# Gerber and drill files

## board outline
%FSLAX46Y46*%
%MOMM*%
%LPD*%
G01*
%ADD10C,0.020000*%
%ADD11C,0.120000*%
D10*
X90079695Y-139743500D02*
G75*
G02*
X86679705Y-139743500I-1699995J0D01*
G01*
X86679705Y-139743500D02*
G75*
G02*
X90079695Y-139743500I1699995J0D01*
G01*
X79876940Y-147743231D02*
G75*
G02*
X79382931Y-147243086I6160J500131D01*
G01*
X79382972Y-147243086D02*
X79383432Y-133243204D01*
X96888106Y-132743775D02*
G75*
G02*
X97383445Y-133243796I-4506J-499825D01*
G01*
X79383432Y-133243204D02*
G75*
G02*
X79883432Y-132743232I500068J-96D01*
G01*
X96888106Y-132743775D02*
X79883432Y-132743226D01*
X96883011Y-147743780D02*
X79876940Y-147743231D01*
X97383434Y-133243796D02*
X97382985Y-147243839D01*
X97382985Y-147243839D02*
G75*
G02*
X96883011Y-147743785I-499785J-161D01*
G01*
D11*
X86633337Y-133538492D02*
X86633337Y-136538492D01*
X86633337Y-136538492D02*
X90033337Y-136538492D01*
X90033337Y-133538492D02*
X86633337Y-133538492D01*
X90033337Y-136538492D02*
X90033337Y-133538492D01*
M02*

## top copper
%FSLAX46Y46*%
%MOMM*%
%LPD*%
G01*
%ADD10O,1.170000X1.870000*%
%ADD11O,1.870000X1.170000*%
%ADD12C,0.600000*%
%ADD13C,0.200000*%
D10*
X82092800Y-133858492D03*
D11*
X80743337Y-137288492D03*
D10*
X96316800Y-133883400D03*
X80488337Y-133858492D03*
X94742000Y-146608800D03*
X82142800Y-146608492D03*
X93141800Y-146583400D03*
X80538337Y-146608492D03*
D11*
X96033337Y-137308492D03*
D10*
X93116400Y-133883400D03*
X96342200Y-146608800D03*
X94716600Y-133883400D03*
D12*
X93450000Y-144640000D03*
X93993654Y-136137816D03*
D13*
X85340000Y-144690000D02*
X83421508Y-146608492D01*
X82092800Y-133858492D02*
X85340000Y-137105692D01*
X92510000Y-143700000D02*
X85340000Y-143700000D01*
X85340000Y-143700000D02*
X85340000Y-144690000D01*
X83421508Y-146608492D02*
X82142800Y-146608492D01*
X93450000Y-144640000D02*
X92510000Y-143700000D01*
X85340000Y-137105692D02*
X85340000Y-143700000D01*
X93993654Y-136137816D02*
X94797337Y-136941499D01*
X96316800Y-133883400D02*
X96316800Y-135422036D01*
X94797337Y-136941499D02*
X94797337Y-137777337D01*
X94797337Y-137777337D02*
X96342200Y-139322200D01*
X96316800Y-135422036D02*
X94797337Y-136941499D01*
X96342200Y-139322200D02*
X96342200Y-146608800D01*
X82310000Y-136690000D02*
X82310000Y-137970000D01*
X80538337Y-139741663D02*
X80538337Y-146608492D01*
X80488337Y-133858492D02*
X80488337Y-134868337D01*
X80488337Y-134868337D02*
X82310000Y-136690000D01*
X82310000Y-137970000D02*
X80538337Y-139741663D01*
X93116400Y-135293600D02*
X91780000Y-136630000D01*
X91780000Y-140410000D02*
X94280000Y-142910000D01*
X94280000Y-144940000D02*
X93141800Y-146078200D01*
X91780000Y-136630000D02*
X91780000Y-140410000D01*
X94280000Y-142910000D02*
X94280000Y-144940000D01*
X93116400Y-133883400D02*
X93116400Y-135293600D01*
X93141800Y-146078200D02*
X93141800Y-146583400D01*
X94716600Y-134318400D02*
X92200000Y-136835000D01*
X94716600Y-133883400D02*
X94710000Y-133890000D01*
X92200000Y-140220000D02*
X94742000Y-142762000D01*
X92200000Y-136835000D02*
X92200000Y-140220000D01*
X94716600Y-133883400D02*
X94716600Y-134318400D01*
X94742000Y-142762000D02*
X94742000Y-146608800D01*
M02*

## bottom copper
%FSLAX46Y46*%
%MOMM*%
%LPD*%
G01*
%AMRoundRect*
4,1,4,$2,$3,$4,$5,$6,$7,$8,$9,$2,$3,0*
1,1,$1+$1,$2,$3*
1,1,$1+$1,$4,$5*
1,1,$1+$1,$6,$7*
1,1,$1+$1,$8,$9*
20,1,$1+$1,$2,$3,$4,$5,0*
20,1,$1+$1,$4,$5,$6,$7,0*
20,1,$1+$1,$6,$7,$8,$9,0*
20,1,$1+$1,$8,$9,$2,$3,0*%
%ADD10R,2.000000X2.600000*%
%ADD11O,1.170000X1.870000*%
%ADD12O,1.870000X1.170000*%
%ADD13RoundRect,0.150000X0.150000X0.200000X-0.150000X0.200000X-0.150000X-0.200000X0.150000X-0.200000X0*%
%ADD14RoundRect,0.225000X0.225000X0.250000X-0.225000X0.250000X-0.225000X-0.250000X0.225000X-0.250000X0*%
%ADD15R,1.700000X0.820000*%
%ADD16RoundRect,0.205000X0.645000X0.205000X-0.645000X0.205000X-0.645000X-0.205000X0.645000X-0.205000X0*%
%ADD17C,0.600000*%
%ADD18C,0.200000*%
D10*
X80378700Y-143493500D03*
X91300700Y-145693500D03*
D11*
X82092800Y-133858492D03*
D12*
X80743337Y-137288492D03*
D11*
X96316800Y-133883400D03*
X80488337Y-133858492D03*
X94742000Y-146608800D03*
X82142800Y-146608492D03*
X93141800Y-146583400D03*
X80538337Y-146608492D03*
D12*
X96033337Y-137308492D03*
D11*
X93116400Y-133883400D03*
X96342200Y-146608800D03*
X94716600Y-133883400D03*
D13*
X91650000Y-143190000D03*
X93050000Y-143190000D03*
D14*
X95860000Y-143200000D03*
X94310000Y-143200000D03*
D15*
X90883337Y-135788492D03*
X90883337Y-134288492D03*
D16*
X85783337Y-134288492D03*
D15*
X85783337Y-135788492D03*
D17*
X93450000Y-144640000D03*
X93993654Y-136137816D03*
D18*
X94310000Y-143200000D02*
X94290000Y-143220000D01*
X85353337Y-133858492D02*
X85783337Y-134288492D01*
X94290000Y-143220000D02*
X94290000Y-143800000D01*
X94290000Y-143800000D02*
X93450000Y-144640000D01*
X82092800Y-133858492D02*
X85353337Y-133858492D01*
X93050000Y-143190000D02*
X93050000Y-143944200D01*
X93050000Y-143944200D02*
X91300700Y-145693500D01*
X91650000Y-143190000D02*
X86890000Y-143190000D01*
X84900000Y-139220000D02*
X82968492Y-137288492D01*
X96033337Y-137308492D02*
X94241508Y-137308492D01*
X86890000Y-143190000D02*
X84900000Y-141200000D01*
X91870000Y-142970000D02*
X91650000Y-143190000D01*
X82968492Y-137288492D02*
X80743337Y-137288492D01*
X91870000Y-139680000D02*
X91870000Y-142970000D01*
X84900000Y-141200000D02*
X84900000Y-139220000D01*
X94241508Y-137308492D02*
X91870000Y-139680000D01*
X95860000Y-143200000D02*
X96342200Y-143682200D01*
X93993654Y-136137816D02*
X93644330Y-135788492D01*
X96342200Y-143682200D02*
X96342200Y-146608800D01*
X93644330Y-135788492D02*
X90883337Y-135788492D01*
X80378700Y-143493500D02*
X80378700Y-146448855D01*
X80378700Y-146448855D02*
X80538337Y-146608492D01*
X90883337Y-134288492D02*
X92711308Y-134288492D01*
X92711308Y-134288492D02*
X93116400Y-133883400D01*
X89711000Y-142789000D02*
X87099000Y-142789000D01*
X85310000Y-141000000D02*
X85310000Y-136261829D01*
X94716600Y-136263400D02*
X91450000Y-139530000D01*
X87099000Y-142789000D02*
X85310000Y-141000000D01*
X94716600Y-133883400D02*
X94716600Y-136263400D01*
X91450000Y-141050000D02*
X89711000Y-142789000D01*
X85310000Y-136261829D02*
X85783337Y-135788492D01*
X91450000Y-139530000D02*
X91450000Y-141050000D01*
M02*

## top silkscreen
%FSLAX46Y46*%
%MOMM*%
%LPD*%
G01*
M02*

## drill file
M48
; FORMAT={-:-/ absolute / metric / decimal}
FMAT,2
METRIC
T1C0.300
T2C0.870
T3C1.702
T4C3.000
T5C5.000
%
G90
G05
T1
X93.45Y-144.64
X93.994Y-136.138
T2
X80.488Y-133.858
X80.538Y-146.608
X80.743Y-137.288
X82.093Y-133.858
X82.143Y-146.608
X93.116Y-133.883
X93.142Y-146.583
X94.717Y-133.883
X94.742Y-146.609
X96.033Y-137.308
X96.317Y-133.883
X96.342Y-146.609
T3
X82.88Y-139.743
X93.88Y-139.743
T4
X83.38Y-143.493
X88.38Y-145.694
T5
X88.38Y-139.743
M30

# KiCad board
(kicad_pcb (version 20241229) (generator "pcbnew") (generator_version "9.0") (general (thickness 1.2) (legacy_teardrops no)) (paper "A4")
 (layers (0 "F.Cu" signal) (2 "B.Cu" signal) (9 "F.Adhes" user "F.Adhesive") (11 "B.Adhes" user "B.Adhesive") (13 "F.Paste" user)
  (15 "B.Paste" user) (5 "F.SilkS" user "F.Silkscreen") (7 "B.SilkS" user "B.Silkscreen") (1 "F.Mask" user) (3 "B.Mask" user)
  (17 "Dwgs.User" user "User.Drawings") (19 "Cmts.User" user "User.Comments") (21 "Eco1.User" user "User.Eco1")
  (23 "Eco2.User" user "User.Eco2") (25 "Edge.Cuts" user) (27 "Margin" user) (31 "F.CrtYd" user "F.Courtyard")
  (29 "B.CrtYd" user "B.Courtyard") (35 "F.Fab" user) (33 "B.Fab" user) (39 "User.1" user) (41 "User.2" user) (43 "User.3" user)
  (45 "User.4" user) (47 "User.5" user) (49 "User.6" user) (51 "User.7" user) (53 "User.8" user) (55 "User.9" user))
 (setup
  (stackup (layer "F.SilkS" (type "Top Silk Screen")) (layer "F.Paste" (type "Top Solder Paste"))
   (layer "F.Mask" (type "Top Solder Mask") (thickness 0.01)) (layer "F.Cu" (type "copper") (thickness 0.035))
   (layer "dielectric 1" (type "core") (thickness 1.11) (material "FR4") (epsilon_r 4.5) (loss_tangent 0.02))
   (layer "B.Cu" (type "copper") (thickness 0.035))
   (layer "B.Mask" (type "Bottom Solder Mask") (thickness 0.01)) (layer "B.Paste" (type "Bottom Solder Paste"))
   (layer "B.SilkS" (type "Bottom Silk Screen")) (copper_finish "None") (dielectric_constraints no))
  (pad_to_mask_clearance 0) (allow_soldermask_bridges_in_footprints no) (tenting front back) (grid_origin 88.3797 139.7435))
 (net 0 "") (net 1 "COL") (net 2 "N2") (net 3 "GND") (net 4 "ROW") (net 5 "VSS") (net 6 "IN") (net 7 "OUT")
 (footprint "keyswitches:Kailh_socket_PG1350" (layer "F.Cu") (at 88.3797 139.7435)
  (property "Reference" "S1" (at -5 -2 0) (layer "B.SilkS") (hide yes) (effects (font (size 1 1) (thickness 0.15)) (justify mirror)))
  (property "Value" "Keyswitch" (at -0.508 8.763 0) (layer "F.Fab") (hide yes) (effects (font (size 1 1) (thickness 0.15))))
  (pad "" np_thru_hole circle (at -5.5 0) (size 1.7018 1.7018) (drill 1.7018) (layers "*.Cu" "*.Mask"))
  (pad "" np_thru_hole circle (at -5 3.75) (size 3 3) (drill 3) (layers "*.Cu" "*.Mask"))
  (pad "" np_thru_hole circle (at 0 0) (size 5 5) (drill 5) (layers "*.Cu" "*.Mask"))
  (pad "" np_thru_hole circle (at 0 5.95) (size 3 3) (drill 3) (layers "*.Cu" "*.Mask"))
  (pad "" np_thru_hole circle (at 5.5 0) (size 1.7018 1.7018) (drill 1.7018) (layers "*.Cu" "*.Mask"))
  (pad "1" smd rect (at -8.001 3.75) (size 2 2.6) (layers "B.Cu" "B.Mask" "B.Paste") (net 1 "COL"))
  (pad "2" smd rect (at 2.921 5.95) (size 2 2.6) (layers "B.Cu" "B.Mask" "B.Paste") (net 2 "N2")))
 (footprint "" (layer "F.Cu") (at 82.0928 133.858492 90)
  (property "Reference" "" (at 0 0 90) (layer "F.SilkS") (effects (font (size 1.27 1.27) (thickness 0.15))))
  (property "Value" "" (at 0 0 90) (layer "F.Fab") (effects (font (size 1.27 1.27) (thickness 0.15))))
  (pad "" thru_hole oval (at 0 0 180) (size 1.17 1.87) (drill 0.87) (layers "*.Cu" "*.Mask") (remove_unused_layers no) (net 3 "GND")))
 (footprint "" (layer "F.Cu") (at 80.743337 137.288492 180)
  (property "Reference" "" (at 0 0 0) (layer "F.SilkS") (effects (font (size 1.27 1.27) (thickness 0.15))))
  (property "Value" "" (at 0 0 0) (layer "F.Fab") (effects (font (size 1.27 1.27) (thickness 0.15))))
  (pad "" thru_hole oval (at 0 0 270) (size 1.17 1.87) (drill 0.87) (layers "*.Cu" "*.Mask") (remove_unused_layers no) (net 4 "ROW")))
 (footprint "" (layer "F.Cu") (at 96.3168 133.8834)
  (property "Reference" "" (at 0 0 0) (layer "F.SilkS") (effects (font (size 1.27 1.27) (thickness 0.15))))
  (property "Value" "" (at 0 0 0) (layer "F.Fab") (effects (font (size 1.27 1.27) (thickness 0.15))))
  (pad "" thru_hole oval (at 0 0 180) (size 1.17 1.87) (drill 0.87) (layers "*.Cu" "*.Mask") (remove_unused_layers no) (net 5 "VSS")))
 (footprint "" (layer "F.Cu") (at 80.488337 133.858492)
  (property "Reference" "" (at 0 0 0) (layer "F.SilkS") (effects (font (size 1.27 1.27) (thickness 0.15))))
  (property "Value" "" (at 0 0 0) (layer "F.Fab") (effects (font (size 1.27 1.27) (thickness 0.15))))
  (pad "" thru_hole oval (at 0 0 180) (size 1.17 1.87) (drill 0.87) (layers "*.Cu" "*.Mask") (remove_unused_layers no) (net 1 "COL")))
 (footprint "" (layer "F.Cu") (at 94.742 146.6088)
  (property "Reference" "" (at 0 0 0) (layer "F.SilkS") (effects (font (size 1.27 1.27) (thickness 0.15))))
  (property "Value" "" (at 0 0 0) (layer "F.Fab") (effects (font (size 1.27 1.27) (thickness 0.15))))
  (pad "" thru_hole oval (at 0 0 180) (size 1.17 1.87) (drill 0.87) (layers "*.Cu" "*.Mask") (remove_unused_layers no) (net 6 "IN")))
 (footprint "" (layer "F.Cu") (at 82.1428 146.608492 90)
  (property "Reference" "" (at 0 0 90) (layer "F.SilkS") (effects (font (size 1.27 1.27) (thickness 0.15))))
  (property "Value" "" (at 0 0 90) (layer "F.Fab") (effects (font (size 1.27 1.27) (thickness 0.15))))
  (pad "" thru_hole oval (at 0 0 180) (size 1.17 1.87) (drill 0.87) (layers "*.Cu" "*.Mask") (remove_unused_layers no) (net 3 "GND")))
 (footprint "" (layer "F.Cu") (at 93.1418 146.5834)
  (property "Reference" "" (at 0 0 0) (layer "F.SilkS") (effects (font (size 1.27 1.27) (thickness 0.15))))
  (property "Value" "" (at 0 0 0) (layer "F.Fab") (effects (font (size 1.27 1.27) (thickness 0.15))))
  (pad "" thru_hole oval (at 0 0 180) (size 1.17 1.87) (drill 0.87) (layers "*.Cu" "*.Mask") (remove_unused_layers no) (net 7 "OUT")))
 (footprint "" (layer "F.Cu") (at 80.538337 146.608492)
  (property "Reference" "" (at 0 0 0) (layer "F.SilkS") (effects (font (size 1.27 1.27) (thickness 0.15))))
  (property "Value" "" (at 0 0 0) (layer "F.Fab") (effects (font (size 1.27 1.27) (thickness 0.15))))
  (pad "" thru_hole oval (at 0 0 180) (size 1.17 1.87) (drill 0.87) (layers "*.Cu" "*.Mask") (remove_unused_layers no) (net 1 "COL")))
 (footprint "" (layer "F.Cu") (at 96.033337 137.308492 180)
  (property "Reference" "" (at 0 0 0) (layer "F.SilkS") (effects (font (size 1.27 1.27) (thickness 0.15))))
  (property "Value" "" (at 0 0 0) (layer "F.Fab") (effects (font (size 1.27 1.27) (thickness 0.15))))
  (pad "" thru_hole oval (at 0 0 270) (size 1.17 1.87) (drill 0.87) (layers "*.Cu" "*.Mask") (remove_unused_layers no) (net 4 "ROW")))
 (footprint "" (layer "F.Cu") (at 93.1164 133.8834)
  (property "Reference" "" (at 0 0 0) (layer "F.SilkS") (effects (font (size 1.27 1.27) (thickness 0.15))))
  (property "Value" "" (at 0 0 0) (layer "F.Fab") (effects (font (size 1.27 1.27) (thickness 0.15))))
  (pad "" thru_hole oval (at 0 0 180) (size 1.17 1.87) (drill 0.87) (layers "*.Cu" "*.Mask") (remove_unused_layers no) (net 7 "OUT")))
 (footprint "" (layer "F.Cu") (at 96.3422 146.6088)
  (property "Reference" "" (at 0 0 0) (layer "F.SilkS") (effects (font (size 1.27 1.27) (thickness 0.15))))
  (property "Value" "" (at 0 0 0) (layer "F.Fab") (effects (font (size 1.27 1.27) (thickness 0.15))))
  (pad "" thru_hole oval (at 0 0 180) (size 1.17 1.87) (drill 0.87) (layers "*.Cu" "*.Mask") (remove_unused_layers no) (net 5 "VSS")))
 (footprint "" (layer "F.Cu") (at 94.7166 133.8834)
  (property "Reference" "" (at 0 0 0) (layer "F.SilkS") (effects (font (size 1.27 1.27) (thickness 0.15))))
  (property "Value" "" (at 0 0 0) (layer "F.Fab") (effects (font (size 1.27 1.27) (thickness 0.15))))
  (pad "" thru_hole oval (at 0 0 180) (size 1.17 1.87) (drill 0.87) (layers "*.Cu" "*.Mask") (remove_unused_layers no) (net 6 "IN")))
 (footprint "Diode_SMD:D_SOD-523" (layer "B.Cu") (at 92.35 143.19)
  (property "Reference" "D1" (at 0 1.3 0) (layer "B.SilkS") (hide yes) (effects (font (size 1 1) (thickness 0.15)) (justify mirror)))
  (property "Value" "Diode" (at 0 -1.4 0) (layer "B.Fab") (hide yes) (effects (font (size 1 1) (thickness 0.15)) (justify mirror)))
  (pad "1" smd roundrect (at -0.7 0 180) (size 0.6 0.7) (layers "B.Cu" "B.Mask" "B.Paste") (roundrect_rratio 0.25) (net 4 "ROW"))
  (pad "2" smd roundrect (at 0.7 0 180) (size 0.6 0.7) (layers "B.Cu" "B.Mask" "B.Paste") (roundrect_rratio 0.25) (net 2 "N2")))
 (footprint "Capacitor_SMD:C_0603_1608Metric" (layer "B.Cu") (at 95.085 143.2 180)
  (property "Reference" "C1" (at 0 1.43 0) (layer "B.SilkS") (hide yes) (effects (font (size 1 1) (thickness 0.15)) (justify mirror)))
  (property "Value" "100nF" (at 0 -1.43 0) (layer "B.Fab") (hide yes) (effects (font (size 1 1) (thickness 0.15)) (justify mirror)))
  (pad "1" smd roundrect (at -0.775 0 180) (size 0.9 0.95) (layers "B.Cu" "B.Mask" "B.Paste") (roundrect_rratio 0.25) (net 5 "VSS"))
  (pad "2" smd roundrect (at 0.775 0 180) (size 0.9 0.95) (layers "B.Cu" "B.Mask" "B.Paste") (roundrect_rratio 0.25) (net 3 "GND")))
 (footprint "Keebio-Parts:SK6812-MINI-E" (layer "B.Cu") (at 88.333337 135.038492 180)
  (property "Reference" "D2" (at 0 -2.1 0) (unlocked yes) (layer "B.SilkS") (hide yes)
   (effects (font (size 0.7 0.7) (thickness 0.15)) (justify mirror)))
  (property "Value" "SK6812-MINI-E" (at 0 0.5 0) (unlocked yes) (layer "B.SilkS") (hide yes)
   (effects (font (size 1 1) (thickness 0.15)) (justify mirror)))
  (fp_line (start 1.7 1.5) (end 1.7 -1.5) (stroke (width 0.12) (type solid)) (layer "Edge.Cuts"))
  (fp_line (start 1.7 -1.5) (end -1.7 -1.5) (stroke (width 0.12) (type solid)) (layer "Edge.Cuts"))
  (fp_line (start -1.7 1.5) (end 1.7 1.5) (stroke (width 0.12) (type solid)) (layer "Edge.Cuts"))
  (fp_line (start -1.7 -1.5) (end -1.7 1.5) (stroke (width 0.12) (type solid)) (layer "Edge.Cuts"))
  (pad "1" smd rect (at -2.55 -0.75 180) (size 1.7 0.82) (layers "B.Cu" "B.Mask" "B.Paste") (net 5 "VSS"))
  (pad "2" smd rect (at -2.55 0.75 180) (size 1.7 0.82) (layers "B.Cu" "B.Mask" "B.Paste") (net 7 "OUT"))
  (pad "3" smd roundrect (at 2.55 0.75 180) (size 1.7 0.82) (layers "B.Cu" "B.Mask" "B.Paste") (roundrect_rratio 0.25) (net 3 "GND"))
  (pad "4" smd rect (at 2.55 -0.75 180) (size 1.7 0.82) (layers "B.Cu" "B.Mask" "B.Paste") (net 6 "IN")))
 (gr_circle (center 88.3797 139.7435) (end 90.068769 139.551067) (stroke (width 0.02) (type default)) (fill no) (layer "Edge.Cuts"))
 (gr_arc (start 79.87694 147.743231) (mid 79.527287 147.594577) (end 79.382972 147.243086) (stroke (width 0.02) (type default))
  (layer "Edge.Cuts"))
 (gr_line (start 79.382972 147.243086) (end 79.383432 133.243204) (stroke (width 0.02) (type default)) (layer "Edge.Cuts"))
 (gr_arc (start 96.888106 132.743775) (mid 97.238703 132.891822) (end 97.383434 133.243796) (stroke (width 0.02) (type default))
  (layer "Edge.Cuts"))
 (gr_arc (start 79.383432 133.243204) (mid 79.529908 132.889689) (end 79.883432 132.743226) (stroke (width 0.02) (type default))
  (layer "Edge.Cuts"))
 (gr_line (start 96.888106 132.743775) (end 79.883432 132.743226) (stroke (width 0.02) (type default)) (layer "Edge.Cuts"))
 (gr_line (start 96.883011 147.74378) (end 79.87694 147.743231) (stroke (width 0.02) (type default)) (layer "Edge.Cuts"))
 (gr_line (start 97.383434 133.243796) (end 97.382985 147.243839) (stroke (width 0.02) (type default)) (layer "Edge.Cuts"))
 (gr_arc (start 97.382985 147.243839) (mid 97.236591 147.597411) (end 96.883011 147.74378) (stroke (width 0.02) (type default))
  (layer "Edge.Cuts"))
 (segment (start 85.34 144.69) (end 83.421508 146.608492) (width 0.2) (layer "F.Cu") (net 3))
 (segment (start 82.0928 133.858492) (end 85.34 137.105692) (width 0.2) (layer "F.Cu") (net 3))
 (segment (start 92.51 143.7) (end 85.34 143.7) (width 0.2) (layer "F.Cu") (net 3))
 (segment (start 85.34 143.7) (end 85.34 144.69) (width 0.2) (layer "F.Cu") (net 3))
 (segment (start 83.421508 146.608492) (end 82.1428 146.608492) (width 0.2) (layer "F.Cu") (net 3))
 (segment (start 93.45 144.64) (end 92.51 143.7) (width 0.2) (layer "F.Cu") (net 3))
 (segment (start 85.34 137.105692) (end 85.34 143.7) (width 0.2) (layer "F.Cu") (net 3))
 (via (at 93.45 144.64) (size 0.6) (drill 0.3) (layers "F.Cu" "B.Cu") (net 3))
 (segment (start 94.31 143.2) (end 94.29 143.22) (width 0.2) (layer "B.Cu") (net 3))
 (segment (start 85.353337 133.858492) (end 85.783337 134.288492) (width 0.2) (layer "B.Cu") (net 3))
 (segment (start 94.29 143.22) (end 94.29 143.8) (width 0.2) (layer "B.Cu") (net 3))
 (segment (start 94.29 143.8) (end 93.45 144.64) (width 0.2) (layer "B.Cu") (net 3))
 (segment (start 82.0928 133.858492) (end 85.353337 133.858492) (width 0.2) (layer "B.Cu") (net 3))
 (segment (start 93.05 143.19) (end 93.05 143.9442) (width 0.2) (layer "B.Cu") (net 2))
 (segment (start 93.05 143.9442) (end 91.3007 145.6935) (width 0.2) (layer "B.Cu") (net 2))
 (segment (start 91.65 143.19) (end 86.89 143.19) (width 0.2) (layer "B.Cu") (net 4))
 (segment (start 84.9 139.22) (end 82.968492 137.288492) (width 0.2) (layer "B.Cu") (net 4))
 (segment (start 96.033337 137.308492) (end 94.241508 137.308492) (width 0.2) (layer "B.Cu") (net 4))
 (segment (start 86.89 143.19) (end 84.9 141.2) (width 0.2) (layer "B.Cu") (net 4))
 (segment (start 91.87 142.97) (end 91.65 143.19) (width 0.2) (layer "B.Cu") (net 4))
 (segment (start 82.968492 137.288492) (end 80.743337 137.288492) (width 0.2) (layer "B.Cu") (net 4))
 (segment (start 91.87 139.68) (end 91.87 142.97) (width 0.2) (layer "B.Cu") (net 4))
 (segment (start 84.9 141.2) (end 84.9 139.22) (width 0.2) (layer "B.Cu") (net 4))
 (segment (start 94.241508 137.308492) (end 91.87 139.68) (width 0.2) (layer "B.Cu") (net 4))
 (segment (start 93.993654 136.137816) (end 94.797337 136.941499) (width 0.2) (layer "F.Cu") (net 5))
 (segment (start 96.3168 133.8834) (end 96.3168 135.422036) (width 0.2) (layer "F.Cu") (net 5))
 (segment (start 94.797337 136.941499) (end 94.797337 137.777337) (width 0.2) (layer "F.Cu") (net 5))
 (segment (start 94.797337 137.777337) (end 96.3422 139.3222) (width 0.2) (layer "F.Cu") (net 5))
 (segment (start 96.3168 135.422036) (end 94.797337 136.941499) (width 0.2) (layer "F.Cu") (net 5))
 (segment (start 96.3422 139.3222) (end 96.3422 146.6088) (width 0.2) (layer "F.Cu") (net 5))
 (via (at 93.993654 136.137816) (size 0.6) (drill 0.3) (layers "F.Cu" "B.Cu") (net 5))
 (segment (start 95.86 143.2) (end 96.3422 143.6822) (width 0.2) (layer "B.Cu") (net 5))
 (segment (start 93.993654 136.137816) (end 93.64433 135.788492) (width 0.2) (layer "B.Cu") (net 5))
 (segment (start 96.3422 143.6822) (end 96.3422 146.6088) (width 0.2) (layer "B.Cu") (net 5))
 (segment (start 93.64433 135.788492) (end 90.883337 135.788492) (width 0.2) (layer "B.Cu") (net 5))
 (segment (start 82.31 136.69) (end 82.31 137.97) (width 0.2) (layer "F.Cu") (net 1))
 (segment (start 80.538337 139.741663) (end 80.538337 146.608492) (width 0.2) (layer "F.Cu") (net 1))
 (segment (start 80.488337 133.858492) (end 80.488337 134.868337) (width 0.2) (layer "F.Cu") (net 1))
 (segment (start 80.488337 134.868337) (end 82.31 136.69) (width 0.2) (layer "F.Cu") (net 1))
 (segment (start 82.31 137.97) (end 80.538337 139.741663) (width 0.2) (layer "F.Cu") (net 1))
 (segment (start 80.3787 143.4935) (end 80.3787 146.448855) (width 0.2) (layer "B.Cu") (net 1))
 (segment (start 80.3787 146.448855) (end 80.538337 146.608492) (width 0.2) (layer "B.Cu") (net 1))
 (segment (start 93.1164 135.2936) (end 91.78 136.63) (width 0.2) (layer "F.Cu") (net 7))
 (segment (start 91.78 140.41) (end 94.28 142.91) (width 0.2) (layer "F.Cu") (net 7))
 (segment (start 94.28 144.94) (end 93.1418 146.0782) (width 0.2) (layer "F.Cu") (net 7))
 (segment (start 91.78 136.63) (end 91.78 140.41) (width 0.2) (layer "F.Cu") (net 7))
 (segment (start 94.28 142.91) (end 94.28 144.94) (width 0.2) (layer "F.Cu") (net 7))
 (segment (start 93.1164 133.8834) (end 93.1164 135.2936) (width 0.2) (layer "F.Cu") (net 7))
 (segment (start 93.1418 146.0782) (end 93.1418 146.5834) (width 0.2) (layer "F.Cu") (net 7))
 (segment (start 90.883337 134.288492) (end 92.711308 134.288492) (width 0.2) (layer "B.Cu") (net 7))
 (segment (start 92.711308 134.288492) (end 93.1164 133.8834) (width 0.2) (layer "B.Cu") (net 7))
 (segment (start 94.7166 134.3184) (end 92.2 136.835) (width 0.2) (layer "F.Cu") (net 6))
 (segment (start 94.7166 133.8834) (end 94.71 133.89) (width 0.2) (layer "F.Cu") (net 6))
 (segment (start 92.2 140.22) (end 94.742 142.762) (width 0.2) (layer "F.Cu") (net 6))
 (segment (start 92.2 136.835) (end 92.2 140.22) (width 0.2) (layer "F.Cu") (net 6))
 (segment (start 94.7166 133.8834) (end 94.7166 134.3184) (width 0.2) (layer "F.Cu") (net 6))
 (segment (start 94.742 142.762) (end 94.742 146.6088) (width 0.2) (layer "F.Cu") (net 6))
 (segment (start 89.711 142.789) (end 87.099 142.789) (width 0.2) (layer "B.Cu") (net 6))
 (segment (start 85.31 141) (end 85.31 136.261829) (width 0.2) (layer "B.Cu") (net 6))
 (segment (start 94.7166 136.2634) (end 91.45 139.53) (width 0.2) (layer "B.Cu") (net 6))
 (segment (start 87.099 142.789) (end 85.31 141) (width 0.2) (layer "B.Cu") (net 6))
 (segment (start 94.7166 133.8834) (end 94.7166 136.2634) (width 0.2) (layer "B.Cu") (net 6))
 (segment (start 91.45 141.05) (end 89.711 142.789) (width 0.2) (layer "B.Cu") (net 6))
 (segment (start 85.31 136.261829) (end 85.783337 135.788492) (width 0.2) (layer "B.Cu") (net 6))
 (segment (start 91.45 139.53) (end 91.45 141.05) (width 0.2) (layer "B.Cu") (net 6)))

